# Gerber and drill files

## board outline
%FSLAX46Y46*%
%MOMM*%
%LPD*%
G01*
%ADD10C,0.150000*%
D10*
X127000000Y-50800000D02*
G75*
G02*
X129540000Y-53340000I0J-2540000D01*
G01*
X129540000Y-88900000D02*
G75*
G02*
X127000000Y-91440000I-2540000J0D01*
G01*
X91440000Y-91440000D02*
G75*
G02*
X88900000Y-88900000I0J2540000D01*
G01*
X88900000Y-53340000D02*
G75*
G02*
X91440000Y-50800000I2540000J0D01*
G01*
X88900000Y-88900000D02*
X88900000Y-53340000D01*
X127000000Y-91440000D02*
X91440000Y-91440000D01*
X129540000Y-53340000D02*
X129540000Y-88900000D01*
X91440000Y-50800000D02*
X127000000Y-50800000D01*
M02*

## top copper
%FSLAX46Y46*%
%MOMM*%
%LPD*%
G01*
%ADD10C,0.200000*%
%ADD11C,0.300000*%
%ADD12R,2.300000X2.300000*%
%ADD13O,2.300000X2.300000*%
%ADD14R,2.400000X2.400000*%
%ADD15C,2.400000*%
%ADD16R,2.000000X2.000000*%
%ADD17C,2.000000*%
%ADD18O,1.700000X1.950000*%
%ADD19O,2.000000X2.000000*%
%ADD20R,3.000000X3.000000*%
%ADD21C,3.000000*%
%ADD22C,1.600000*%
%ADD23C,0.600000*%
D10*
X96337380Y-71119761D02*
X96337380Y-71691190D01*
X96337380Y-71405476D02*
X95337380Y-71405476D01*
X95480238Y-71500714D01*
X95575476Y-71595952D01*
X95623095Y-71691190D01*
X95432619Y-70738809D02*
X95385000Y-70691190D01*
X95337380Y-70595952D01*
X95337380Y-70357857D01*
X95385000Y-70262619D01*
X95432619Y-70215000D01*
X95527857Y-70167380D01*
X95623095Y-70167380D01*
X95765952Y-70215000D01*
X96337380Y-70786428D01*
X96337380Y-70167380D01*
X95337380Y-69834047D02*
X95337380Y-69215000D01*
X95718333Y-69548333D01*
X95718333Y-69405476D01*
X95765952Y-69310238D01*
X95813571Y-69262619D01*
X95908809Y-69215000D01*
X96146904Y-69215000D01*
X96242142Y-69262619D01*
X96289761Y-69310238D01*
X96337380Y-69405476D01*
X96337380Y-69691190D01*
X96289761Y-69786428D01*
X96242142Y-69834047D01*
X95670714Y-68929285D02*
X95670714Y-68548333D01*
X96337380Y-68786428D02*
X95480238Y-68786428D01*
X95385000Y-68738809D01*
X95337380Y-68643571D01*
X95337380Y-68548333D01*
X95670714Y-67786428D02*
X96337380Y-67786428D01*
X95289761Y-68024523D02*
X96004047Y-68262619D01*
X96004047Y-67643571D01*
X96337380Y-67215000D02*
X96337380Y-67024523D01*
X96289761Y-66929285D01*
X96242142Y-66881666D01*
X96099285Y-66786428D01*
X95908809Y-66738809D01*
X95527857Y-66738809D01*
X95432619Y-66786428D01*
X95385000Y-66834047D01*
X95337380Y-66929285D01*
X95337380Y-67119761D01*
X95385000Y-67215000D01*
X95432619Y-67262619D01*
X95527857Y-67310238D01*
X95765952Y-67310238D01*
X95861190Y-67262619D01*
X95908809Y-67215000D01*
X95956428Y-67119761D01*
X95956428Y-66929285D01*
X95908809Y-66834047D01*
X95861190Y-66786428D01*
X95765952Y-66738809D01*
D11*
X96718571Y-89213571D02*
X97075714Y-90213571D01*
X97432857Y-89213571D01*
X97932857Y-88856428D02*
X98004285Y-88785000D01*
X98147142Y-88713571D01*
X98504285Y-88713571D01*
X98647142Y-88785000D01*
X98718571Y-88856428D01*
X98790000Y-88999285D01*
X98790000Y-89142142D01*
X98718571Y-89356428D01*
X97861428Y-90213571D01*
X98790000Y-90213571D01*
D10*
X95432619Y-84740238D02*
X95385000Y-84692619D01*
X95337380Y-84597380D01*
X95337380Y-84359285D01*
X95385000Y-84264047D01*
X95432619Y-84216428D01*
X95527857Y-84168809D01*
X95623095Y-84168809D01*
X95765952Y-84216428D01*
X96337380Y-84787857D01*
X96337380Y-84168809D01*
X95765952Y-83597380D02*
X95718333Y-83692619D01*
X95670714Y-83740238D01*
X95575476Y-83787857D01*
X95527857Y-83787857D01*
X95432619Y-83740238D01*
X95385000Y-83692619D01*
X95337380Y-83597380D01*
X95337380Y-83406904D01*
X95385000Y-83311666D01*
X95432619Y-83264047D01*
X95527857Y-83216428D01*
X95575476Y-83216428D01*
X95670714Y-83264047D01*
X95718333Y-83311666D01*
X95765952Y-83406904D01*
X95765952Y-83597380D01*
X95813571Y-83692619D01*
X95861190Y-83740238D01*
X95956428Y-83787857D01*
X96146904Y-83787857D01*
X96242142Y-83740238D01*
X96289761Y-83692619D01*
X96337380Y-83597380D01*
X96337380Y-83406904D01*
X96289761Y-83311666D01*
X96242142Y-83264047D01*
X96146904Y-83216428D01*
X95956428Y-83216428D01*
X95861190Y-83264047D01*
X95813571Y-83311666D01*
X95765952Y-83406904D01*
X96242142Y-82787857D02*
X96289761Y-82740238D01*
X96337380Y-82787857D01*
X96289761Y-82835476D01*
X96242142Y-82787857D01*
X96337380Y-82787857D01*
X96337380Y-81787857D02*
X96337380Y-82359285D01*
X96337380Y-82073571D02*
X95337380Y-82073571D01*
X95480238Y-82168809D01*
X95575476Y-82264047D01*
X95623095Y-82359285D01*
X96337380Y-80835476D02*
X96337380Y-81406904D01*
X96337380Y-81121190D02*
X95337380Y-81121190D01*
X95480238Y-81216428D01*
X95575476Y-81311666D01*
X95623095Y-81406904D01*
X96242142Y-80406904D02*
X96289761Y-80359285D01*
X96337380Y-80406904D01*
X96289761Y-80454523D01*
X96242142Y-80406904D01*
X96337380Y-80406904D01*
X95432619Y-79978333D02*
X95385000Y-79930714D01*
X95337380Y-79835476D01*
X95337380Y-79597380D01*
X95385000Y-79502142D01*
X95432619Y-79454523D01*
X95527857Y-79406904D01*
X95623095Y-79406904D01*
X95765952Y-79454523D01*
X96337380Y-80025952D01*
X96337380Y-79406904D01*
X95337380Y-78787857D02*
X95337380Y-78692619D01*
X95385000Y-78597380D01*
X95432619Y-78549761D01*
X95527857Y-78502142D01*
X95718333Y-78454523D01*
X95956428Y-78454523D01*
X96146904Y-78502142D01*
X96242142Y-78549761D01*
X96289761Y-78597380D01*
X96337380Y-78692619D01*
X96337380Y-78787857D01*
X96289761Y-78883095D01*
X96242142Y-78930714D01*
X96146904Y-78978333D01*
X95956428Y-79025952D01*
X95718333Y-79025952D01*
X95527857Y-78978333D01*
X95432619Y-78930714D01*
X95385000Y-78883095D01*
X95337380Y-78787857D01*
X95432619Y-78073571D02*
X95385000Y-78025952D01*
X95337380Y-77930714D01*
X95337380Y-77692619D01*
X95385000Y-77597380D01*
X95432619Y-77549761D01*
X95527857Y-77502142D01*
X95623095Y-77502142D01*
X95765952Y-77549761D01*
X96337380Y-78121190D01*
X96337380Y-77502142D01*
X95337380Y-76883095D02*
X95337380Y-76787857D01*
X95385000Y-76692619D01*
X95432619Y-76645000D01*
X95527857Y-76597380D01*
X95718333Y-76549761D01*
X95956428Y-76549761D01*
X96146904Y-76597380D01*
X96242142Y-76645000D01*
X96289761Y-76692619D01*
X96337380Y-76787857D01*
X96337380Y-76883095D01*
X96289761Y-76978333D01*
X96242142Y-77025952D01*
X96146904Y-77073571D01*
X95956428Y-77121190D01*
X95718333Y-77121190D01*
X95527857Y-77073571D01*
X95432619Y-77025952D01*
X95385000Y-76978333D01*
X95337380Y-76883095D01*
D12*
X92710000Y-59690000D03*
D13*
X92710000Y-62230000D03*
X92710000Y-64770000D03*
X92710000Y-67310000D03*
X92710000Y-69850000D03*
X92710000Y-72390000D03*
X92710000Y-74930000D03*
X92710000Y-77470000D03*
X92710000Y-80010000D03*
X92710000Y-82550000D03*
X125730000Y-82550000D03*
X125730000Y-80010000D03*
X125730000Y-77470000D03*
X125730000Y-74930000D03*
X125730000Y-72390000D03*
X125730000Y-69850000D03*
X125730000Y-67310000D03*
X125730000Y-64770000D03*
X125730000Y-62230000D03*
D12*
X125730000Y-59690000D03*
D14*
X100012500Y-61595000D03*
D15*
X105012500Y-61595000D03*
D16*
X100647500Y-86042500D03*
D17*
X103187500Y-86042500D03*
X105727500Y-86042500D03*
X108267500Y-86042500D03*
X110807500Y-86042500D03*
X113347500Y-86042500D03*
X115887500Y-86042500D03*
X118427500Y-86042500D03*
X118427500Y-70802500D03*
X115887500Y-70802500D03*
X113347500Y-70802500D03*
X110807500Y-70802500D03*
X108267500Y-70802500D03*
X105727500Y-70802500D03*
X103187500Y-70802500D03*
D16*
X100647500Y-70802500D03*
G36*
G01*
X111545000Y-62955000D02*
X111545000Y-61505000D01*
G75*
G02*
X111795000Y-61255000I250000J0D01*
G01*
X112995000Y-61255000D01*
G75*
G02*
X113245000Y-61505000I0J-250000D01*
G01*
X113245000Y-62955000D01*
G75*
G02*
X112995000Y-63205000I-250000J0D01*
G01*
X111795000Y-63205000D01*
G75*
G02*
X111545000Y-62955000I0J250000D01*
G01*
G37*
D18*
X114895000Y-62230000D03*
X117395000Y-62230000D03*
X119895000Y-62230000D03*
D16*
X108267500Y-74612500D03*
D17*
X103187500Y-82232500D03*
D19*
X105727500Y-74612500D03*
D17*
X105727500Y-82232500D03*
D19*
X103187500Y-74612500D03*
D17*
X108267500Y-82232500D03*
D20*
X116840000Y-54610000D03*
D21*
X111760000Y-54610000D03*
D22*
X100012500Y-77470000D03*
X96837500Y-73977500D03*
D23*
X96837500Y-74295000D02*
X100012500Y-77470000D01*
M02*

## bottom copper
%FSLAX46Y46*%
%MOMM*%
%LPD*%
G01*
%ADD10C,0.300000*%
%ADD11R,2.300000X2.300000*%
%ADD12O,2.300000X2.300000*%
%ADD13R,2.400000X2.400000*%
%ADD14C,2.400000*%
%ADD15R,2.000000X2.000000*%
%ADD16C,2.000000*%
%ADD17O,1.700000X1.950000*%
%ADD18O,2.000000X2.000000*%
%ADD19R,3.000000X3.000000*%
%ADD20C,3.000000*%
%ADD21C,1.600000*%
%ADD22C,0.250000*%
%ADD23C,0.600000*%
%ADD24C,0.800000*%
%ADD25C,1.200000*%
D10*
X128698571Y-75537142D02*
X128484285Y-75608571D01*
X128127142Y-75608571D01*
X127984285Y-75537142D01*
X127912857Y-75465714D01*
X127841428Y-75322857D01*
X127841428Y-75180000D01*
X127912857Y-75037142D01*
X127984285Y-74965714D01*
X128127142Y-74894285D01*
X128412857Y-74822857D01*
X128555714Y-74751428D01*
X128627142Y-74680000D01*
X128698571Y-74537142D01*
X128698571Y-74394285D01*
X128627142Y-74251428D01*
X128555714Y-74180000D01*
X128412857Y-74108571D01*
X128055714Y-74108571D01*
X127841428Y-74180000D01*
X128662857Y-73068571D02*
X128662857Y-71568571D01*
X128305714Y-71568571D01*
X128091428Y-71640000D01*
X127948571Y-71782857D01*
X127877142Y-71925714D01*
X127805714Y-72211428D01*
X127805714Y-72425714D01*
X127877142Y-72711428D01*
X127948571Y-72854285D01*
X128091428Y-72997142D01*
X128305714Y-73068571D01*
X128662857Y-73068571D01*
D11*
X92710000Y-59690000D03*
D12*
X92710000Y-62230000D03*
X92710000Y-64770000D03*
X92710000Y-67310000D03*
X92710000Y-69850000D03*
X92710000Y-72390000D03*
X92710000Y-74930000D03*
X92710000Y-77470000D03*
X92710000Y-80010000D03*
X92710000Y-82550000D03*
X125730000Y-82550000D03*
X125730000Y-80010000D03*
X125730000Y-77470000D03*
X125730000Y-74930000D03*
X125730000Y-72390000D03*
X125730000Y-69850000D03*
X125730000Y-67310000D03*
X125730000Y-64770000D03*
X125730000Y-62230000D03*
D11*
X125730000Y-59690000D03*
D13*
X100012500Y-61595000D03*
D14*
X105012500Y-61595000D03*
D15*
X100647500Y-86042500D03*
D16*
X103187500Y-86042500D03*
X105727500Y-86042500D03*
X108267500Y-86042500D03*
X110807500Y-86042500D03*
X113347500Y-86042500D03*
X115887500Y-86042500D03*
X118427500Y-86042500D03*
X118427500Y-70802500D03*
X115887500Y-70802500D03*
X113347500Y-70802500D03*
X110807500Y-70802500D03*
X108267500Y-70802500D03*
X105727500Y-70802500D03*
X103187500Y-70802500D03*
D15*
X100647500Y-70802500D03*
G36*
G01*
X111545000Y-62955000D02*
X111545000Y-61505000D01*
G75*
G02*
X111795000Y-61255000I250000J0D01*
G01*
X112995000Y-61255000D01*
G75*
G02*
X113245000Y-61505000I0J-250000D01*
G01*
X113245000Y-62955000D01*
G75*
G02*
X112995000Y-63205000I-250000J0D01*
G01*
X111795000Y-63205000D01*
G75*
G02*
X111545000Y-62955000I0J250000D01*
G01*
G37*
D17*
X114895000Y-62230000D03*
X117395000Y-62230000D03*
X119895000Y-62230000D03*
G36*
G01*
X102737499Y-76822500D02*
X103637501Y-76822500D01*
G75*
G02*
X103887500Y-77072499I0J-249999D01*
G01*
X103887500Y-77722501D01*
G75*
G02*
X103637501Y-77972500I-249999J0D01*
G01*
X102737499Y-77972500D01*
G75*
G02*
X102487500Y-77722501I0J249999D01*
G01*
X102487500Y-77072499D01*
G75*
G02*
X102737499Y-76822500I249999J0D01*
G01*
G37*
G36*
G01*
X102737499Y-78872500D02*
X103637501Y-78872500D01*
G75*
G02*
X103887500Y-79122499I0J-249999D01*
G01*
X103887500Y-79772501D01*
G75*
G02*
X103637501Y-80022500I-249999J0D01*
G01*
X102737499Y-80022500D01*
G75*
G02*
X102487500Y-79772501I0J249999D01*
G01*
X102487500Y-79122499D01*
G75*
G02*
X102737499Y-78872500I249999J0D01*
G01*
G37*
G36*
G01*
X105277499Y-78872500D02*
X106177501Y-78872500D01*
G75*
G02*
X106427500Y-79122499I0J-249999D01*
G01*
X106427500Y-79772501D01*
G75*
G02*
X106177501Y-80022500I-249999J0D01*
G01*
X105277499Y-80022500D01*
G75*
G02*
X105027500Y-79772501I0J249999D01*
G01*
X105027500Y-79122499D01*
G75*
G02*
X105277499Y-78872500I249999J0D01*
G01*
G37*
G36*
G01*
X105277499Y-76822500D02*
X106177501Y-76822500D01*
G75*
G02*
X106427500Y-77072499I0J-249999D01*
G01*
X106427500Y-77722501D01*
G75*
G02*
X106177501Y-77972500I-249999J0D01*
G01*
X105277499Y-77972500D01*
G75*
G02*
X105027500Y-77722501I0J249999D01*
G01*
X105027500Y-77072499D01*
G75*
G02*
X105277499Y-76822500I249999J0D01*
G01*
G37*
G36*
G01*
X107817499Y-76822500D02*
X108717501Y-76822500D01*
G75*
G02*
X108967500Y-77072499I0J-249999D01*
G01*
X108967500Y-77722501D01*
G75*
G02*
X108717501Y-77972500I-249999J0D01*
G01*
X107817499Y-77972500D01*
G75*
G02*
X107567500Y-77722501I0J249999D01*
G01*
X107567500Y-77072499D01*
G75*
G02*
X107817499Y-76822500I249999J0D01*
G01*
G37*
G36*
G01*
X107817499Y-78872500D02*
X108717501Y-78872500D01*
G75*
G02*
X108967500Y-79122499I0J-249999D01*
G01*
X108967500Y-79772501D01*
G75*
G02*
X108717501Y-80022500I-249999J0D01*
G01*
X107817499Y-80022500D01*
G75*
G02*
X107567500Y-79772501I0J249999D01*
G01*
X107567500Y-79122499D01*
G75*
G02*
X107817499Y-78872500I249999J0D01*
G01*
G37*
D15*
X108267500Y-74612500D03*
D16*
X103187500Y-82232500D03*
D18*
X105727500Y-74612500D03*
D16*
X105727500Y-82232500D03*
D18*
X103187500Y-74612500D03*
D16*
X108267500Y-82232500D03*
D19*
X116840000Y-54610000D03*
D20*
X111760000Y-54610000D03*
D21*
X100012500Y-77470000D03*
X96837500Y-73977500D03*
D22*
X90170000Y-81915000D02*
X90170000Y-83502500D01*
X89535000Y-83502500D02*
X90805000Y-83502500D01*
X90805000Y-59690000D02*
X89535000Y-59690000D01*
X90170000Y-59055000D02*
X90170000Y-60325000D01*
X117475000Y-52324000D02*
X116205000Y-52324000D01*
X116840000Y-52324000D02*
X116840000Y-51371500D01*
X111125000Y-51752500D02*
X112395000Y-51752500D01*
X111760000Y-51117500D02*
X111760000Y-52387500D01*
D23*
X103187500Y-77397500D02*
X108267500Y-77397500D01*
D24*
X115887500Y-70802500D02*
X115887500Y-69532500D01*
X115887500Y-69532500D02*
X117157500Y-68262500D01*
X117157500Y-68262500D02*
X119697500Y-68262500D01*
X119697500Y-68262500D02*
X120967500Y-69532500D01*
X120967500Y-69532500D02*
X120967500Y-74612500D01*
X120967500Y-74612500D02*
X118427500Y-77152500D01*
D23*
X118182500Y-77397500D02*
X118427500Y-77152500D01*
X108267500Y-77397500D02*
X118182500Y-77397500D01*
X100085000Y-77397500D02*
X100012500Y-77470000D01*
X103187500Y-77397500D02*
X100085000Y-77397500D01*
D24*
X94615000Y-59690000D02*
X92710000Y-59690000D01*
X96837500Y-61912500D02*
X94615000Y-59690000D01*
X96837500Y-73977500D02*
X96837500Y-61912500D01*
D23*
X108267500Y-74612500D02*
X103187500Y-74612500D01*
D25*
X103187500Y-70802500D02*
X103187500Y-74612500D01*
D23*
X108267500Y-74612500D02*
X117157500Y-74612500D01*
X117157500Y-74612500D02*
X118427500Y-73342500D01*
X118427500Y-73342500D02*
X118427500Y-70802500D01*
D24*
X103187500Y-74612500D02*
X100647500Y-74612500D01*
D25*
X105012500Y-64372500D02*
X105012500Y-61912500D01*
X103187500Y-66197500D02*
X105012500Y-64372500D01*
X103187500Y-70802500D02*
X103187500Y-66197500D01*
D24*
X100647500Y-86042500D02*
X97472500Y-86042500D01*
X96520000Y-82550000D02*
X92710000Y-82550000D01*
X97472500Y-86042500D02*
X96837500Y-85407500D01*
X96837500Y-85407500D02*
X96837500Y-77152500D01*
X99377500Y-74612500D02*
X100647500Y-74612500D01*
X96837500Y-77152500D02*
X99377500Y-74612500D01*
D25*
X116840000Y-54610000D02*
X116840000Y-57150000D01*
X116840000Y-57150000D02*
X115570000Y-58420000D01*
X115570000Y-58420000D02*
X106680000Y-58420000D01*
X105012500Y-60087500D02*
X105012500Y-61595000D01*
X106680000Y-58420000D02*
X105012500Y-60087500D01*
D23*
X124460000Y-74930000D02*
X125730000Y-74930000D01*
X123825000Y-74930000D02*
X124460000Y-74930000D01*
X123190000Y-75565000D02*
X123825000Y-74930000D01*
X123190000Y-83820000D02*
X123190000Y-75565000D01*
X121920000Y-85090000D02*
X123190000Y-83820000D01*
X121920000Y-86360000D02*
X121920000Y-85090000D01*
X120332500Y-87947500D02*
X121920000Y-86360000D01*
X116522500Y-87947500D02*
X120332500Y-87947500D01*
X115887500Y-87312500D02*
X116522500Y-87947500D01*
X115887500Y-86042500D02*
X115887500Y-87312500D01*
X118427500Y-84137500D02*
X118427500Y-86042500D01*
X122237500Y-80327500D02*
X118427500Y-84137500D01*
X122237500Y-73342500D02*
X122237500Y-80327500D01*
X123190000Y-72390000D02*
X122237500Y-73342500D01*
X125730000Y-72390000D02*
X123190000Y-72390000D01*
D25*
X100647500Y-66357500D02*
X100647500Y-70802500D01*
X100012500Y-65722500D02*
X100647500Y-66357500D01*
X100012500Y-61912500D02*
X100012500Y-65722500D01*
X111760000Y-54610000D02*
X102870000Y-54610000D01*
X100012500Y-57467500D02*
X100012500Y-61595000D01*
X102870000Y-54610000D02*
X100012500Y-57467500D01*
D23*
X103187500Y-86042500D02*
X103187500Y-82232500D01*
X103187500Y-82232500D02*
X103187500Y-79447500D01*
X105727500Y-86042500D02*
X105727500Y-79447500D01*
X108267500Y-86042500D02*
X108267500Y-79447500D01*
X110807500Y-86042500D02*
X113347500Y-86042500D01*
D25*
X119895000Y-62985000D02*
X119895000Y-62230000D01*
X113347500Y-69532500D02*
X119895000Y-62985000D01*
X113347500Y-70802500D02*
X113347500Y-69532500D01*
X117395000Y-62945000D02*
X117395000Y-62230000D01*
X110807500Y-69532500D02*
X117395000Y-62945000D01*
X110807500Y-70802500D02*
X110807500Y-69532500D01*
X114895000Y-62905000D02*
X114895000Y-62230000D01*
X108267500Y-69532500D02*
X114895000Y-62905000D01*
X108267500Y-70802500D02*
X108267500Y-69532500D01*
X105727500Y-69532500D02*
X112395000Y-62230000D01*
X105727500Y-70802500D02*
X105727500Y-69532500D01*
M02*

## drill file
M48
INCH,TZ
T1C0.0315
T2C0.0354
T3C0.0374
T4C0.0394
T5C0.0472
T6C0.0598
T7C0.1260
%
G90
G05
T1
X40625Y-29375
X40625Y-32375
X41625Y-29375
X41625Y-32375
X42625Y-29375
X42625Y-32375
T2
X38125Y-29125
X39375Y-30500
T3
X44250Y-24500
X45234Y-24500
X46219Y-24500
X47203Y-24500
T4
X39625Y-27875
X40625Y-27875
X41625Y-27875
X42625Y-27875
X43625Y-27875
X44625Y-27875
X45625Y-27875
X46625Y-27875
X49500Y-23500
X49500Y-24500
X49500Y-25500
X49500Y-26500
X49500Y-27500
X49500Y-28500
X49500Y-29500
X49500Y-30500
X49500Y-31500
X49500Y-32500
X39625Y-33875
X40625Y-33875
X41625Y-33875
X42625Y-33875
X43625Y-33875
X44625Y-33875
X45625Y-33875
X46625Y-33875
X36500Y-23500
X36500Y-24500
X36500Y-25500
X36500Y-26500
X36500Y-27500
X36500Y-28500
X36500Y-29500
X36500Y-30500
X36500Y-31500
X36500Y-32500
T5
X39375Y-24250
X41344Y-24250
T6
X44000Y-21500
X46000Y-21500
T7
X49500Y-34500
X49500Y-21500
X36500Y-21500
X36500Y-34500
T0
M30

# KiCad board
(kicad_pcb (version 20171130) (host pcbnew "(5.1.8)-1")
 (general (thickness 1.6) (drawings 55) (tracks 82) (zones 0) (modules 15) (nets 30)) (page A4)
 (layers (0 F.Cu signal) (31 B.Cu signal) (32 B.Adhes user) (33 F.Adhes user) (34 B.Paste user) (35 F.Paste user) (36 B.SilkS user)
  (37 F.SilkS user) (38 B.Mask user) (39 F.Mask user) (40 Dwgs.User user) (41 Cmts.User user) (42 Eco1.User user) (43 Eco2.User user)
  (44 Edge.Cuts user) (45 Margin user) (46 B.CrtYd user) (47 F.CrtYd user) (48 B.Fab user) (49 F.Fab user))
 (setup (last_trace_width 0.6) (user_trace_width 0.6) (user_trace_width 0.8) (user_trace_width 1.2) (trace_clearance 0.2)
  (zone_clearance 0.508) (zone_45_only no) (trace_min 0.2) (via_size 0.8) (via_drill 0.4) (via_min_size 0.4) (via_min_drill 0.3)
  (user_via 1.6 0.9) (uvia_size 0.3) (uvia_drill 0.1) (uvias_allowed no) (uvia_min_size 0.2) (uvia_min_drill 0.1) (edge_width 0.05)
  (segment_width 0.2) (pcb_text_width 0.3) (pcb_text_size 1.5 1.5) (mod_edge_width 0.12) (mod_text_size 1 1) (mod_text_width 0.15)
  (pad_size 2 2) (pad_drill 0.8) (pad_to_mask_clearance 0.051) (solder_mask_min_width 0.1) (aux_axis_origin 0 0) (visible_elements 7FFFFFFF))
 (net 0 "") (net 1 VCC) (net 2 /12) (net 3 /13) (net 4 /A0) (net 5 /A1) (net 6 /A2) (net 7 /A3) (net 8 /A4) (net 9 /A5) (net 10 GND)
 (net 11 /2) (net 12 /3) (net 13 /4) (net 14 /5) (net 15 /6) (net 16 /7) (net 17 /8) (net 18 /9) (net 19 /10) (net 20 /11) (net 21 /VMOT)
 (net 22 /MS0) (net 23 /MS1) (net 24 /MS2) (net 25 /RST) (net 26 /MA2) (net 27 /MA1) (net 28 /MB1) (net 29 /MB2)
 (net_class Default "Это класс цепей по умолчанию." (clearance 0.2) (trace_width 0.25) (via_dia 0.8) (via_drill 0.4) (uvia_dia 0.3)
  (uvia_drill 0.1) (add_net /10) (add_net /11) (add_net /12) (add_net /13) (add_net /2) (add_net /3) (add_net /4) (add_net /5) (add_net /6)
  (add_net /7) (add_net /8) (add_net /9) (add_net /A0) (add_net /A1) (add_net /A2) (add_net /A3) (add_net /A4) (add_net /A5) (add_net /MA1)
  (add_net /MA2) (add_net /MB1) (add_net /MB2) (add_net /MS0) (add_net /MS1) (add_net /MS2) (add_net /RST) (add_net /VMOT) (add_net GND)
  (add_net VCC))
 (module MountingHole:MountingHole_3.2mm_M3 (layer F.Cu) (at 92.71 54.61)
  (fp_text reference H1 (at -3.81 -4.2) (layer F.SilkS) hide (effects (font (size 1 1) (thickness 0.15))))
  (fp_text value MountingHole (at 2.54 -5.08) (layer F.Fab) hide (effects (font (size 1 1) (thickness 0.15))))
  (pad 1 np_thru_hole circle (at 0 0) (size 3.2 3.2) (drill 3.2) (layers *.Cu *.Mask)))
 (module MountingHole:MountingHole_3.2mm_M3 (layer F.Cu) (at 92.71 87.63)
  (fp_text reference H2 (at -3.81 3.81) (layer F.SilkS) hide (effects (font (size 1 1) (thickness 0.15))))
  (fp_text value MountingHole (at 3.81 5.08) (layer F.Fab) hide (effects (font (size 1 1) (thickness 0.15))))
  (pad 1 np_thru_hole circle (at 0 0) (size 3.2 3.2) (drill 3.2) (layers *.Cu *.Mask)))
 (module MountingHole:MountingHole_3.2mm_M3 (layer F.Cu) (at 125.73 54.61)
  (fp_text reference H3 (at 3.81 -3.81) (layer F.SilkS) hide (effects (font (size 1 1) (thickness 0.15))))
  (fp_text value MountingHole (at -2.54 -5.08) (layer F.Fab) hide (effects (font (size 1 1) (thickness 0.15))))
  (pad 1 np_thru_hole circle (at 0 0) (size 3.2 3.2) (drill 3.2) (layers *.Cu *.Mask)))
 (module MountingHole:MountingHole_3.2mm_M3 (layer F.Cu) (at 125.73 87.63)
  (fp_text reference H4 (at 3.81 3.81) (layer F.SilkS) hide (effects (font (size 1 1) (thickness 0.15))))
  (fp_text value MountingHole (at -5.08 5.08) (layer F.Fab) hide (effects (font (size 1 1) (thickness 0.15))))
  (pad 1 np_thru_hole circle (at 0 0) (size 3.2 3.2) (drill 3.2) (layers *.Cu *.Mask)))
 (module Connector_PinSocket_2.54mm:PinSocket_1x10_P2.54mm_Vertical (layer F.Cu) (at 92.71 59.69)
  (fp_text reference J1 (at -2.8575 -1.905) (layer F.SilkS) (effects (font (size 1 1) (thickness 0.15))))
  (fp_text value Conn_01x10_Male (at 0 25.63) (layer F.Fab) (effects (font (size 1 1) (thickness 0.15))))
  (pad 1 thru_hole rect (at 0 0) (size 2.3 2.3) (drill 1) (layers *.Cu *.Mask) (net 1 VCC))
  (pad 2 thru_hole oval (at 0 2.54) (size 2.3 2.3) (drill 1) (layers *.Cu *.Mask) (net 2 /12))
  (pad 3 thru_hole oval (at 0 5.08) (size 2.3 2.3) (drill 1) (layers *.Cu *.Mask) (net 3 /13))
  (pad 4 thru_hole oval (at 0 7.62) (size 2.3 2.3) (drill 1) (layers *.Cu *.Mask) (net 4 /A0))
  (pad 5 thru_hole oval (at 0 10.16) (size 2.3 2.3) (drill 1) (layers *.Cu *.Mask) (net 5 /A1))
  (pad 6 thru_hole oval (at 0 12.7) (size 2.3 2.3) (drill 1) (layers *.Cu *.Mask) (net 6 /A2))
  (pad 7 thru_hole oval (at 0 15.24) (size 2.3 2.3) (drill 1) (layers *.Cu *.Mask) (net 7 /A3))
  (pad 8 thru_hole oval (at 0 17.78) (size 2.3 2.3) (drill 1) (layers *.Cu *.Mask) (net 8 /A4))
  (pad 9 thru_hole oval (at 0 20.32) (size 2.3 2.3) (drill 1) (layers *.Cu *.Mask) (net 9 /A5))
  (pad 10 thru_hole oval (at 0 22.86) (size 2.3 2.3) (drill 1) (layers *.Cu *.Mask) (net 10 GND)))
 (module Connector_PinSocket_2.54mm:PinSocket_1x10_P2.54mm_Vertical (layer F.Cu) (at 125.73 59.69)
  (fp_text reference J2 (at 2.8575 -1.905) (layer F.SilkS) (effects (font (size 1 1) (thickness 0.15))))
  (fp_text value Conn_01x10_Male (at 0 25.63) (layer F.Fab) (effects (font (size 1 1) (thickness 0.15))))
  (pad 10 thru_hole oval (at 0 22.86) (size 2.3 2.3) (drill 1) (layers *.Cu *.Mask) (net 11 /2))
  (pad 9 thru_hole oval (at 0 20.32) (size 2.3 2.3) (drill 1) (layers *.Cu *.Mask) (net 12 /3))
  (pad 8 thru_hole oval (at 0 17.78) (size 2.3 2.3) (drill 1) (layers *.Cu *.Mask) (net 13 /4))
  (pad 7 thru_hole oval (at 0 15.24) (size 2.3 2.3) (drill 1) (layers *.Cu *.Mask) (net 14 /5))
  (pad 6 thru_hole oval (at 0 12.7) (size 2.3 2.3) (drill 1) (layers *.Cu *.Mask) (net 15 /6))
  (pad 5 thru_hole oval (at 0 10.16) (size 2.3 2.3) (drill 1) (layers *.Cu *.Mask) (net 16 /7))
  (pad 4 thru_hole oval (at 0 7.62) (size 2.3 2.3) (drill 1) (layers *.Cu *.Mask) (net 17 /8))
  (pad 3 thru_hole oval (at 0 5.08) (size 2.3 2.3) (drill 1) (layers *.Cu *.Mask) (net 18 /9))
  (pad 2 thru_hole oval (at 0 2.54) (size 2.3 2.3) (drill 1) (layers *.Cu *.Mask) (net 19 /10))
  (pad 1 thru_hole rect (at 0 0) (size 2.3 2.3) (drill 1) (layers *.Cu *.Mask) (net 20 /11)))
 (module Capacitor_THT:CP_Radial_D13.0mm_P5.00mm (layer F.Cu) (at 100.0125 61.595)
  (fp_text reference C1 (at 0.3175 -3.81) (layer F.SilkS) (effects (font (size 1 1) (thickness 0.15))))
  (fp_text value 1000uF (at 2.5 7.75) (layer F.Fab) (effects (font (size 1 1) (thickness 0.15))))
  (pad 1 thru_hole rect (at 0 0) (size 2.4 2.4) (drill 1.2) (layers *.Cu *.Mask) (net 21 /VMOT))
  (pad 2 thru_hole circle (at 5 0) (size 2.4 2.4) (drill 1.2) (layers *.Cu *.Mask) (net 10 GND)))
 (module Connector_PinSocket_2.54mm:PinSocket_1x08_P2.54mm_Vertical (layer F.Cu) (at 100.6475 86.0425 90)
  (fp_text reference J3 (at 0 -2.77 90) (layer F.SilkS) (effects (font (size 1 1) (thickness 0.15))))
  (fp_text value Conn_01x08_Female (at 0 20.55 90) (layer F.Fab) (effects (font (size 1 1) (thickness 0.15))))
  (pad 1 thru_hole rect (at 0 0 90) (size 2 2) (drill 1) (layers *.Cu *.Mask) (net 10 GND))
  (pad 2 thru_hole circle (at 0 2.54 90) (size 2 2) (drill 1) (layers *.Cu *.Mask) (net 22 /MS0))
  (pad 3 thru_hole circle (at 0 5.08 90) (size 2 2) (drill 1) (layers *.Cu *.Mask) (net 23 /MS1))
  (pad 4 thru_hole circle (at 0 7.62 90) (size 2 2) (drill 1) (layers *.Cu *.Mask) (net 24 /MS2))
  (pad 5 thru_hole circle (at 0 10.16 90) (size 2 2) (drill 1) (layers *.Cu *.Mask) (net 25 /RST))
  (pad 6 thru_hole circle (at 0 12.7 90) (size 2 2) (drill 1) (layers *.Cu *.Mask) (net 25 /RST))
  (pad 7 thru_hole circle (at 0 15.24 90) (size 2 2) (drill 1) (layers *.Cu *.Mask) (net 14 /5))
  (pad 8 thru_hole circle (at 0 17.78 90) (size 2 2) (drill 1) (layers *.Cu *.Mask) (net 15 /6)))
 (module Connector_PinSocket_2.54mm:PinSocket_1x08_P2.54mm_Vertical (layer F.Cu) (at 100.6475 70.8025 90)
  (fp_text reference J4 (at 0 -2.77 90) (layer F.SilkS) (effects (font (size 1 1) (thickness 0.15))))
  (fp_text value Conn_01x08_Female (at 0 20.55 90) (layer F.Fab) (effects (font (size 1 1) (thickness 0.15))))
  (pad 8 thru_hole circle (at 0 17.78 90) (size 2 2) (drill 1) (layers *.Cu *.Mask) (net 10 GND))
  (pad 7 thru_hole circle (at 0 15.24 90) (size 2 2) (drill 1) (layers *.Cu *.Mask) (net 1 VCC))
  (pad 6 thru_hole circle (at 0 12.7 90) (size 2 2) (drill 1) (layers *.Cu *.Mask) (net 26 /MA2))
  (pad 5 thru_hole circle (at 0 10.16 90) (size 2 2) (drill 1) (layers *.Cu *.Mask) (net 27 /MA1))
  (pad 4 thru_hole circle (at 0 7.62 90) (size 2 2) (drill 1) (layers *.Cu *.Mask) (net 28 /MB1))
  (pad 3 thru_hole circle (at 0 5.08 90) (size 2 2) (drill 1) (layers *.Cu *.Mask) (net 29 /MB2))
  (pad 2 thru_hole circle (at 0 2.54 90) (size 2 2) (drill 1) (layers *.Cu *.Mask) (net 10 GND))
  (pad 1 thru_hole rect (at 0 0 90) (size 2 2) (drill 1) (layers *.Cu *.Mask) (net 21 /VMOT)))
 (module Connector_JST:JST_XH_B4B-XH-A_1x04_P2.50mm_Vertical (layer F.Cu) (at 112.395 62.23)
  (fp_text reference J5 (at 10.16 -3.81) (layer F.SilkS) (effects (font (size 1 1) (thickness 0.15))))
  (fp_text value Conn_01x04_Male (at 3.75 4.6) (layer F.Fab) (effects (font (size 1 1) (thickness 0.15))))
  (pad 1 thru_hole roundrect (at 0 0) (size 1.7 1.95) (drill 0.95) (layers *.Cu *.Mask) (roundrect_rratio 0.1470588235294118) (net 29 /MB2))
  (pad 2 thru_hole oval (at 2.5 0) (size 1.7 1.95) (drill 0.95) (layers *.Cu *.Mask) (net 28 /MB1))
  (pad 3 thru_hole oval (at 5 0) (size 1.7 1.95) (drill 0.95) (layers *.Cu *.Mask) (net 27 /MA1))
  (pad 4 thru_hole oval (at 7.5 0) (size 1.7 1.95) (drill 0.95) (layers *.Cu *.Mask) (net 26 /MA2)))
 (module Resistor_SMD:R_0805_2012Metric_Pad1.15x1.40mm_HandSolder (layer B.Cu) (at 103.1875 78.4225 270)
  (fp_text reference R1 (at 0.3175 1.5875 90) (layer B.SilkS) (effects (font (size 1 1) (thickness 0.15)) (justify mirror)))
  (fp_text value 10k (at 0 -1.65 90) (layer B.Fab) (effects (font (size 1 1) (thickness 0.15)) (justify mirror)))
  (pad 1 smd roundrect (at -1.025 0 270) (size 1.15 1.4) (layers B.Cu B.Paste B.Mask) (roundrect_rratio 0.2173904347826087) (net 1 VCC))
  (pad 2 smd roundrect (at 1.025 0 270) (size 1.15 1.4) (layers B.Cu B.Paste B.Mask) (roundrect_rratio 0.2173904347826087) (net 22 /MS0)))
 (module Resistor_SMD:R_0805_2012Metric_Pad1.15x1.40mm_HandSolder (layer B.Cu) (at 105.7275 78.4225 270)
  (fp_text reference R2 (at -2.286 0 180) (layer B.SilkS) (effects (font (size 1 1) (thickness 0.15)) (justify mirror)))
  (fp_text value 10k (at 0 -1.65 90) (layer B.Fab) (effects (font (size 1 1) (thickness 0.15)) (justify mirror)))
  (pad 2 smd roundrect (at 1.025 0 270) (size 1.15 1.4) (layers B.Cu B.Paste B.Mask) (roundrect_rratio 0.2173904347826087) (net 23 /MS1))
  (pad 1 smd roundrect (at -1.025 0 270) (size 1.15 1.4) (layers B.Cu B.Paste B.Mask) (roundrect_rratio 0.2173904347826087) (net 1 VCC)))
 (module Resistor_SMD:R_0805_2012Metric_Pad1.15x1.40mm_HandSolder (layer B.Cu) (at 108.2675 78.4225 270)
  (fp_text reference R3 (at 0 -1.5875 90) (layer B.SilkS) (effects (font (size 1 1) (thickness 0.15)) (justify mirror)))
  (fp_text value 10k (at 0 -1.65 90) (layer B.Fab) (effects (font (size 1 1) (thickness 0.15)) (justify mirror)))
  (pad 1 smd roundrect (at -1.025 0 270) (size 1.15 1.4) (layers B.Cu B.Paste B.Mask) (roundrect_rratio 0.2173904347826087) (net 1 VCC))
  (pad 2 smd roundrect (at 1.025 0 270) (size 1.15 1.4) (layers B.Cu B.Paste B.Mask) (roundrect_rratio 0.2173904347826087) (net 24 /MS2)))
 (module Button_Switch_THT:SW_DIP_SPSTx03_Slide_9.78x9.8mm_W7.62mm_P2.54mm (layer F.Cu) (at 108.2675 74.6125 270)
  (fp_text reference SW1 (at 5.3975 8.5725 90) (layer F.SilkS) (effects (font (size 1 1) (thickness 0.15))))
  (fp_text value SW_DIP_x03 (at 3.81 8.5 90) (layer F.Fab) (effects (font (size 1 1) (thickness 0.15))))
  (pad 1 thru_hole rect (at 0 0 270) (size 2 2) (drill 0.8) (layers *.Cu *.Mask) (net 10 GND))
  (pad 4 thru_hole circle (at 7.62 5.08 270) (size 2 2) (drill 0.8) (layers *.Cu *.Mask) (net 22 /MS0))
  (pad 2 thru_hole oval (at 0 2.54 270) (size 2 2) (drill 0.8) (layers *.Cu *.Mask) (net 10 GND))
  (pad 5 thru_hole circle (at 7.62 2.54 270) (size 2 2) (drill 0.8) (layers *.Cu *.Mask) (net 23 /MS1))
  (pad 3 thru_hole oval (at 0 5.08 270) (size 2 2) (drill 0.8) (layers *.Cu *.Mask) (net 10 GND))
  (pad 6 thru_hole circle (at 7.62 0 270) (size 2 2) (drill 0.8) (layers *.Cu *.Mask) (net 24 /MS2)))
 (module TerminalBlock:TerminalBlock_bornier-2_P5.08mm (layer F.Cu) (at 116.84 54.61 180)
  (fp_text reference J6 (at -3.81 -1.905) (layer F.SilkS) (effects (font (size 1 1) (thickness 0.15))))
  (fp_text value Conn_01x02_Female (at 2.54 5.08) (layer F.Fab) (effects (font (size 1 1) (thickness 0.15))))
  (pad 1 thru_hole rect (at 0 0 180) (size 3 3) (drill 1.52) (layers *.Cu *.Mask) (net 10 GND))
  (pad 2 thru_hole circle (at 5.08 0 180) (size 3 3) (drill 1.52) (layers *.Cu *.Mask) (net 21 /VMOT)))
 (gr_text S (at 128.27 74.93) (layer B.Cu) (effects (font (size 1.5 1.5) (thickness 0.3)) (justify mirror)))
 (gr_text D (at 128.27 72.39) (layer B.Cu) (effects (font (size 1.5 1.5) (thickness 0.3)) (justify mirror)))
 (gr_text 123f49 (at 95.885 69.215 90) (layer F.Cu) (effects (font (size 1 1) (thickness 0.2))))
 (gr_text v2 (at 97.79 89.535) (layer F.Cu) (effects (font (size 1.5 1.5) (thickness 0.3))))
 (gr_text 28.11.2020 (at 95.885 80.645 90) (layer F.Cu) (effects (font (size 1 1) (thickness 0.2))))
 (gr_arc (start 127 53.34) (end 129.54 53.34) (angle -90) (layer Edge.Cuts) (width 0.15))
 (gr_arc (start 127 88.9) (end 127 91.44) (angle -90) (layer Edge.Cuts) (width 0.15))
 (gr_arc (start 91.44 88.9) (end 88.9 88.9) (angle -90) (layer Edge.Cuts) (width 0.15))
 (gr_arc (start 91.44 53.34) (end 91.44 50.8) (angle -90) (layer Edge.Cuts) (width 0.15))
 (gr_line (start 88.9 88.9) (end 88.9 53.34) (layer Edge.Cuts) (width 0.15))
 (gr_line (start 127 91.44) (end 91.44 91.44) (layer Edge.Cuts) (width 0.15))
 (gr_line (start 129.54 53.34) (end 129.54 88.9) (layer Edge.Cuts) (width 0.15))
 (gr_line (start 91.44 50.8) (end 127 50.8) (layer Edge.Cuts) (width 0.15))
 (segment (start 90.17 81.915) (end 90.17 83.5025) (width 0.25) (layer B.Cu) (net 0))
 (segment (start 89.535 83.5025) (end 90.805 83.5025) (width 0.25) (layer B.Cu) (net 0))
 (segment (start 90.805 59.69) (end 89.535 59.69) (width 0.25) (layer B.Cu) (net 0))
 (segment (start 90.17 59.055) (end 90.17 60.325) (width 0.25) (layer B.Cu) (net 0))
 (segment (start 117.475 52.324) (end 116.205 52.324) (width 0.25) (layer B.Cu) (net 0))
 (segment (start 116.84 52.324) (end 116.84 51.3715) (width 0.25) (layer B.Cu) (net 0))
 (segment (start 111.125 51.7525) (end 112.395 51.7525) (width 0.25) (layer B.Cu) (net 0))
 (segment (start 111.76 51.1175) (end 111.76 52.3875) (width 0.25) (layer B.Cu) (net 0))
 (via (at 100.0125 77.47) (size 1.6) (drill 0.9) (layers F.Cu B.Cu) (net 1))
 (segment (start 103.1875 77.3975) (end 108.2675 77.3975) (width 0.6) (layer B.Cu) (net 1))
 (segment (start 115.8875 70.8025) (end 115.8875 69.5325) (width 0.8) (layer B.Cu) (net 1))
 (segment (start 115.8875 69.5325) (end 117.1575 68.2625) (width 0.8) (layer B.Cu) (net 1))
 (segment (start 117.1575 68.2625) (end 119.6975 68.2625) (width 0.8) (layer B.Cu) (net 1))
 (segment (start 119.6975 68.2625) (end 120.9675 69.5325) (width 0.8) (layer B.Cu) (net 1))
 (segment (start 120.9675 69.5325) (end 120.9675 74.6125) (width 0.8) (layer B.Cu) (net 1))
 (segment (start 120.9675 74.6125) (end 118.4275 77.1525) (width 0.8) (layer B.Cu) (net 1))
 (segment (start 118.1825 77.3975) (end 118.4275 77.1525) (width 0.6) (layer B.Cu) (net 1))
 (segment (start 108.2675 77.3975) (end 118.1825 77.3975) (width 0.6) (layer B.Cu) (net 1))
 (via (at 96.8375 73.9775) (size 1.6) (drill 0.9) (layers F.Cu B.Cu) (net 1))
 (segment (start 100.085 77.3975) (end 100.0125 77.47) (width 0.6) (layer B.Cu) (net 1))
 (segment (start 103.1875 77.3975) (end 100.085 77.3975) (width 0.6) (layer B.Cu) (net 1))
 (segment (start 96.8375 74.295) (end 100.0125 77.47) (width 0.6) (layer F.Cu) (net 1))
 (segment (start 94.615 59.69) (end 92.71 59.69) (width 0.8) (layer B.Cu) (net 1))
 (segment (start 96.8375 61.9125) (end 94.615 59.69) (width 0.8) (layer B.Cu) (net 1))
 (segment (start 96.8375 73.9775) (end 96.8375 61.9125) (width 0.8) (layer B.Cu) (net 1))
 (segment (start 108.2675 74.6125) (end 103.1875 74.6125) (width 0.6) (layer B.Cu) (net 10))
 (segment (start 103.1875 70.8025) (end 103.1875 74.6125) (width 1.2) (layer B.Cu) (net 10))
 (segment (start 108.2675 74.6125) (end 117.1575 74.6125) (width 0.6) (layer B.Cu) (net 10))
 (segment (start 117.1575 74.6125) (end 118.4275 73.3425) (width 0.6) (layer B.Cu) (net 10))
 (segment (start 118.4275 73.3425) (end 118.4275 70.8025) (width 0.6) (layer B.Cu) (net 10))
 (segment (start 103.1875 74.6125) (end 100.6475 74.6125) (width 0.8) (layer B.Cu) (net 10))
 (segment (start 105.0125 64.3725) (end 105.0125 61.9125) (width 1.2) (layer B.Cu) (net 10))
 (segment (start 103.1875 66.1975) (end 105.0125 64.3725) (width 1.2) (layer B.Cu) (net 10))
 (segment (start 103.1875 70.8025) (end 103.1875 66.1975) (width 1.2) (layer B.Cu) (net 10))
 (segment (start 100.6475 86.0425) (end 97.4725 86.0425) (width 0.8) (layer B.Cu) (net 10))
 (segment (start 96.52 82.55) (end 92.71 82.55) (width 0.8) (layer B.Cu) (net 10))
 (segment (start 97.4725 86.0425) (end 96.8375 85.4075) (width 0.8) (layer B.Cu) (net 10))
 (segment (start 96.8375 85.4075) (end 96.8375 77.1525) (width 0.8) (layer B.Cu) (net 10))
 (segment (start 99.3775 74.6125) (end 100.6475 74.6125) (width 0.8) (layer B.Cu) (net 10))
 (segment (start 96.8375 77.1525) (end 99.3775 74.6125) (width 0.8) (layer B.Cu) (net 10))
 (segment (start 116.84 54.61) (end 116.84 57.15) (width 1.2) (layer B.Cu) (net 10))
 (segment (start 116.84 57.15) (end 115.57 58.42) (width 1.2) (layer B.Cu) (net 10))
 (segment (start 115.57 58.42) (end 106.68 58.42) (width 1.2) (layer B.Cu) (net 10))
 (segment (start 105.0125 60.0875) (end 105.0125 61.595) (width 1.2) (layer B.Cu) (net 10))
 (segment (start 106.68 58.42) (end 105.0125 60.0875) (width 1.2) (layer B.Cu) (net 10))
 (segment (start 124.46 74.93) (end 125.73 74.93) (width 0.6) (layer B.Cu) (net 14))
 (segment (start 123.825 74.93) (end 124.46 74.93) (width 0.6) (layer B.Cu) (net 14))
 (segment (start 123.19 75.565) (end 123.825 74.93) (width 0.6) (layer B.Cu) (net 14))
 (segment (start 123.19 83.82) (end 123.19 75.565) (width 0.6) (layer B.Cu) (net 14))
 (segment (start 121.92 85.09) (end 123.19 83.82) (width 0.6) (layer B.Cu) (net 14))
 (segment (start 121.92 86.36) (end 121.92 85.09) (width 0.6) (layer B.Cu) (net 14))
 (segment (start 120.3325 87.9475) (end 121.92 86.36) (width 0.6) (layer B.Cu) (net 14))
 (segment (start 116.5225 87.9475) (end 120.3325 87.9475) (width 0.6) (layer B.Cu) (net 14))
 (segment (start 115.8875 87.3125) (end 116.5225 87.9475) (width 0.6) (layer B.Cu) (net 14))
 (segment (start 115.8875 86.0425) (end 115.8875 87.3125) (width 0.6) (layer B.Cu) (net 14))
 (segment (start 118.4275 84.1375) (end 118.4275 86.0425) (width 0.6) (layer B.Cu) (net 15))
 (segment (start 122.2375 80.3275) (end 118.4275 84.1375) (width 0.6) (layer B.Cu) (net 15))
 (segment (start 122.2375 73.3425) (end 122.2375 80.3275) (width 0.6) (layer B.Cu) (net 15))
 (segment (start 123.19 72.39) (end 122.2375 73.3425) (width 0.6) (layer B.Cu) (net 15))
 (segment (start 125.73 72.39) (end 123.19 72.39) (width 0.6) (layer B.Cu) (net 15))
 (segment (start 100.6475 66.3575) (end 100.6475 70.8025) (width 1.2) (layer B.Cu) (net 21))
 (segment (start 100.0125 65.7225) (end 100.6475 66.3575) (width 1.2) (layer B.Cu) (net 21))
 (segment (start 100.0125 61.9125) (end 100.0125 65.7225) (width 1.2) (layer B.Cu) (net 21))
 (segment (start 111.76 54.61) (end 102.87 54.61) (width 1.2) (layer B.Cu) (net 21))
 (segment (start 100.0125 57.4675) (end 100.0125 61.595) (width 1.2) (layer B.Cu) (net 21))
 (segment (start 102.87 54.61) (end 100.0125 57.4675) (width 1.2) (layer B.Cu) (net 21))
 (segment (start 103.1875 86.0425) (end 103.1875 82.2325) (width 0.6) (layer B.Cu) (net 22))
 (segment (start 103.1875 82.2325) (end 103.1875 79.4475) (width 0.6) (layer B.Cu) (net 22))
 (segment (start 105.7275 86.0425) (end 105.7275 79.4475) (width 0.6) (layer B.Cu) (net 23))
 (segment (start 108.2675 86.0425) (end 108.2675 79.4475) (width 0.6) (layer B.Cu) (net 24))
 (segment (start 110.8075 86.0425) (end 113.3475 86.0425) (width 0.6) (layer B.Cu) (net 25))
 (segment (start 119.895 62.985) (end 119.895 62.23) (width 1.2) (layer B.Cu) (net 26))
 (segment (start 113.3475 69.5325) (end 119.895 62.985) (width 1.2) (layer B.Cu) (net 26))
 (segment (start 113.3475 70.8025) (end 113.3475 69.5325) (width 1.2) (layer B.Cu) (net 26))
 (segment (start 117.395 62.945) (end 117.395 62.23) (width 1.2) (layer B.Cu) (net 27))
 (segment (start 110.8075 69.5325) (end 117.395 62.945) (width 1.2) (layer B.Cu) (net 27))
 (segment (start 110.8075 70.8025) (end 110.8075 69.5325) (width 1.2) (layer B.Cu) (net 27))
 (segment (start 114.895 62.905) (end 114.895 62.23) (width 1.2) (layer B.Cu) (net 28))
 (segment (start 108.2675 69.5325) (end 114.895 62.905) (width 1.2) (layer B.Cu) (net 28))
 (segment (start 108.2675 70.8025) (end 108.2675 69.5325) (width 1.2) (layer B.Cu) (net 28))
 (segment (start 105.7275 69.5325) (end 112.395 62.23) (width 1.2) (layer B.Cu) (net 29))
 (segment (start 105.7275 70.8025) (end 105.7275 69.5325) (width 1.2) (layer B.Cu) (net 29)))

